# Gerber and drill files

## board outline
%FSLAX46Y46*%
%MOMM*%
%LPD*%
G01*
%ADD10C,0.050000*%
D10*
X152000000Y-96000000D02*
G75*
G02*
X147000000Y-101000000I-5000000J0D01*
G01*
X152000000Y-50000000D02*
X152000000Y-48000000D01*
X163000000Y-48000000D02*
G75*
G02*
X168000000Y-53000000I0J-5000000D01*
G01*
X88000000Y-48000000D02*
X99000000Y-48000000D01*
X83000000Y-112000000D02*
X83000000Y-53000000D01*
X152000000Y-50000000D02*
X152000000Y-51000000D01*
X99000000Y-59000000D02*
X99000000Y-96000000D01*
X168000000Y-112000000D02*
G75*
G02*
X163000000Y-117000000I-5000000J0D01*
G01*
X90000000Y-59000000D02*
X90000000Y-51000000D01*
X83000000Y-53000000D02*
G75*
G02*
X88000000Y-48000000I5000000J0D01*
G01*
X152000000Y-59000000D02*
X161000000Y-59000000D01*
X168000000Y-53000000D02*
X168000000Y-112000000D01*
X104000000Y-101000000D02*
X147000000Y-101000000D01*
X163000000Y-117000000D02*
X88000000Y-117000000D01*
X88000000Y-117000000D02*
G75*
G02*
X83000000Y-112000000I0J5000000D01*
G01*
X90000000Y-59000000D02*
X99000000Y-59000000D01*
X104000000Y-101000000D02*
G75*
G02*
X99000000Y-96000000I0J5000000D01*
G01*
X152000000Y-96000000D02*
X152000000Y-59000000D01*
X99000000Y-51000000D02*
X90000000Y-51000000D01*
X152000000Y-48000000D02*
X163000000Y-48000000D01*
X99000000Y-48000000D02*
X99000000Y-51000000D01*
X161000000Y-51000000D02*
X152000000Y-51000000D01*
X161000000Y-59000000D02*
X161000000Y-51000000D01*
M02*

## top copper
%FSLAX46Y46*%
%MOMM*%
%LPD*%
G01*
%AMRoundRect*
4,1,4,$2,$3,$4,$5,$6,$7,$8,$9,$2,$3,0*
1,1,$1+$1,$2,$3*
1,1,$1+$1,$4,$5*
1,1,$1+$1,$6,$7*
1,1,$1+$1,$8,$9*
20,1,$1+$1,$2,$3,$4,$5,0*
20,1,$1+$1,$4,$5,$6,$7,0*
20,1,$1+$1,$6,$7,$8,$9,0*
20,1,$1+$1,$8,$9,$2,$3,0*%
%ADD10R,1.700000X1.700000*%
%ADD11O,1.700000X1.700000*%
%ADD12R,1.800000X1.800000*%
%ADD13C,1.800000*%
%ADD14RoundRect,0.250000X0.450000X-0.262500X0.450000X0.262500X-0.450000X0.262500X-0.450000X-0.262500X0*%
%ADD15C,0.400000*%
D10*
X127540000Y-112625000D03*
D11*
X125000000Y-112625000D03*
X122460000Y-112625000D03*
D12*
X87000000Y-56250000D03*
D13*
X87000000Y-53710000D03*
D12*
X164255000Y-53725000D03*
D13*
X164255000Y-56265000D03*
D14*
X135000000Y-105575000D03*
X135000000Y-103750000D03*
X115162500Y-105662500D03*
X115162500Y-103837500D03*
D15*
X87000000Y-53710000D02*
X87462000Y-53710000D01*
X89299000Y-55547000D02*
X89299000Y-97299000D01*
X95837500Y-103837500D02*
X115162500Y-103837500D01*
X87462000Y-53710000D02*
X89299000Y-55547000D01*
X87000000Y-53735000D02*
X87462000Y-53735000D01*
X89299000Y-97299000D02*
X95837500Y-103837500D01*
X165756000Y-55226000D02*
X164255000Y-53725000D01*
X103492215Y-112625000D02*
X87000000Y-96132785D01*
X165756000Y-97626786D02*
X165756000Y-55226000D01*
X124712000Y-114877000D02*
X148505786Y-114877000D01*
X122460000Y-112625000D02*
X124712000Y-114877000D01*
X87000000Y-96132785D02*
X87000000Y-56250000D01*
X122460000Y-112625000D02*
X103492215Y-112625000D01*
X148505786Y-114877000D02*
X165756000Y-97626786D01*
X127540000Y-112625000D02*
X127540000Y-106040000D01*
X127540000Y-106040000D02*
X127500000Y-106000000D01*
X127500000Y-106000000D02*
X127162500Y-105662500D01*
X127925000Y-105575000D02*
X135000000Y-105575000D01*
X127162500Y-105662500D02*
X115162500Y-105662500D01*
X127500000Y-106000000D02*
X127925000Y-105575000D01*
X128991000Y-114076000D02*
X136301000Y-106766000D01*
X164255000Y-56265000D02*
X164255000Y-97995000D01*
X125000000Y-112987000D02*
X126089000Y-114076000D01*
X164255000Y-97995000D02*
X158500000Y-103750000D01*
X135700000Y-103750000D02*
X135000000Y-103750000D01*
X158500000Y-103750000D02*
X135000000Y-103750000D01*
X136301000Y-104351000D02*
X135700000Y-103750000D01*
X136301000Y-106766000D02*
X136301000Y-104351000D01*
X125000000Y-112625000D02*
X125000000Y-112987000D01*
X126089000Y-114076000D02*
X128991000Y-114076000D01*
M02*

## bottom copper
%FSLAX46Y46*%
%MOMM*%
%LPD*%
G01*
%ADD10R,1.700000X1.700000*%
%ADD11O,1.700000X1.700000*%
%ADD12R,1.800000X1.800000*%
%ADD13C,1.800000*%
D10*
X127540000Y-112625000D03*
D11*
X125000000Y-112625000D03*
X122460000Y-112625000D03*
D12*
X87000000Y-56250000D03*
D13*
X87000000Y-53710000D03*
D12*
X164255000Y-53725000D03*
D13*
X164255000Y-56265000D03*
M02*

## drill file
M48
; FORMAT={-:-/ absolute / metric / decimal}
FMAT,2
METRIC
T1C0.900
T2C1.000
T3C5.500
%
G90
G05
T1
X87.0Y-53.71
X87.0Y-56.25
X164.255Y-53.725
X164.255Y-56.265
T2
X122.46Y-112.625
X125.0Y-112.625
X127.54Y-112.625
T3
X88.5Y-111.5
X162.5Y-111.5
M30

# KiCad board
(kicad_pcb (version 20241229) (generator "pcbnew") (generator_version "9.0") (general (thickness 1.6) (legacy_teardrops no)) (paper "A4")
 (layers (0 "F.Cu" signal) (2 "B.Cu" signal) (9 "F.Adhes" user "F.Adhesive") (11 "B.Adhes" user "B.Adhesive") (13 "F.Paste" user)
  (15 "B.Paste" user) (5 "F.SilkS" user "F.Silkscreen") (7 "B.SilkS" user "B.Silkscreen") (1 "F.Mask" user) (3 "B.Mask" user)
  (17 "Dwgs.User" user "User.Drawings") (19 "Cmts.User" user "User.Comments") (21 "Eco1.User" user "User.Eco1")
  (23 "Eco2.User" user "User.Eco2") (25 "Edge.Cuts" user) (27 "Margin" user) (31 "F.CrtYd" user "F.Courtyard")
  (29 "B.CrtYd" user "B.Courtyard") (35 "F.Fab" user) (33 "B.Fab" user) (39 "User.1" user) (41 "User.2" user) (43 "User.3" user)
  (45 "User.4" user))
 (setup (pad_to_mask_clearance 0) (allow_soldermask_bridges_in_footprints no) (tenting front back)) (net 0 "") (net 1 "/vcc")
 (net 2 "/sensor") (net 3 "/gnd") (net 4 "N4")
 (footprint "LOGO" (layer "F.Cu") (at 92.75 75.25 90)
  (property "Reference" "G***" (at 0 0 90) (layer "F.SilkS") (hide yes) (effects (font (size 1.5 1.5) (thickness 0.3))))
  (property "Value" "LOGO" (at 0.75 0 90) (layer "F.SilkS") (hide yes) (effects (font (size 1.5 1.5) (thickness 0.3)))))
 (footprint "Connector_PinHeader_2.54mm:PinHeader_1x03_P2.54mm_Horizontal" (layer "F.Cu") (at 127.54 112.625 -90)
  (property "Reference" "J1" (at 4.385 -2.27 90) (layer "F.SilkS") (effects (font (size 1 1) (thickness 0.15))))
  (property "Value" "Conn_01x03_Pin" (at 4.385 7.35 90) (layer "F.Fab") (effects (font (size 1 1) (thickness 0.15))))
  (pad "1" thru_hole rect (at 0 0 270) (size 1.7 1.7) (drill 1) (layers "*.Cu" "*.Mask") (remove_unused_layers no) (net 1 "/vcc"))
  (pad "2" thru_hole oval (at 0 2.54 270) (size 1.7 1.7) (drill 1) (layers "*.Cu" "*.Mask") (remove_unused_layers no) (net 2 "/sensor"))
  (pad "3" thru_hole oval (at 0 5.08 270) (size 1.7 1.7) (drill 1) (layers "*.Cu" "*.Mask") (remove_unused_layers no) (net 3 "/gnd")))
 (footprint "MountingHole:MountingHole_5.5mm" (layer "F.Cu") (at 88.5 111.5)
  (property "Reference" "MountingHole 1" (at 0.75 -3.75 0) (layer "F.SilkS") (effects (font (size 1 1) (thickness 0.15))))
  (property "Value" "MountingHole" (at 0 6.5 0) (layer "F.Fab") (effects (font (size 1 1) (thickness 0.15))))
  (pad "" np_thru_hole circle (at 0 0) (size 5.5 5.5) (drill 5.5) (layers "*.Cu" "*.Mask")))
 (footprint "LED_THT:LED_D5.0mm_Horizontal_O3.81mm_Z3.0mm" (layer "F.Cu") (at 87 56.25 90)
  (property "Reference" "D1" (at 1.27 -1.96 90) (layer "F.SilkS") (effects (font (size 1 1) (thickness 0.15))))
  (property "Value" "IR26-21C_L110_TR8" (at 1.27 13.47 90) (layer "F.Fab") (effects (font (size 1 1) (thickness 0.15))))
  (pad "1" thru_hole rect (at 0 0 90) (size 1.8 1.8) (drill 0.9) (layers "*.Cu" "*.Mask") (remove_unused_layers no) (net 3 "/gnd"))
  (pad "2" thru_hole circle (at 2.54 0 90) (size 1.8 1.8) (drill 0.9) (layers "*.Cu" "*.Mask") (remove_unused_layers no) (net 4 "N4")))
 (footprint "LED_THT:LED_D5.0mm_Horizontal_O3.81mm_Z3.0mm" (layer "F.Cu") (at 164.255 53.725 -90)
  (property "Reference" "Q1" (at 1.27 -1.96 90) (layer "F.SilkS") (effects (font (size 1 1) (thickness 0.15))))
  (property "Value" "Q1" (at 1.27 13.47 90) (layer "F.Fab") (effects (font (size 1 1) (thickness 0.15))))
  (pad "1" thru_hole rect (at 0 0 270) (size 1.8 1.8) (drill 0.9) (layers "*.Cu" "*.Mask") (remove_unused_layers no) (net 3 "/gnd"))
  (pad "2" thru_hole circle (at 2.54 0 270) (size 1.8 1.8) (drill 0.9) (layers "*.Cu" "*.Mask") (remove_unused_layers no) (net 2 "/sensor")))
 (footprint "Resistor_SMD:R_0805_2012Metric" (layer "F.Cu") (at 135 104.6625 90)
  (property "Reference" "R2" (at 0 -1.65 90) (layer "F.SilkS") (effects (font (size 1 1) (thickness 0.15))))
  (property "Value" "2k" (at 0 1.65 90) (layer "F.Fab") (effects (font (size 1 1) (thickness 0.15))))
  (pad "1" smd roundrect (at -0.9125 0 90) (size 1.025 1.4) (layers "F.Cu" "F.Mask" "F.Paste") (roundrect_rratio 0.243902) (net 1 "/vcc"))
  (pad "2" smd roundrect (at 0.9125 0 90) (size 1.025 1.4) (layers "F.Cu" "F.Mask" "F.Paste") (roundrect_rratio 0.243902) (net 2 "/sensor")))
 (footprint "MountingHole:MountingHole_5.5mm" (layer "F.Cu") (at 162.5 111.5)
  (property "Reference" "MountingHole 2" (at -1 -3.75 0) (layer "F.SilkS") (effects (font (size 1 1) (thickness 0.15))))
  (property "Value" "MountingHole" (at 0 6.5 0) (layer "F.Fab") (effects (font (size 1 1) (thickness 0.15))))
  (pad "" np_thru_hole circle (at 0 0) (size 5.5 5.5) (drill 5.5) (layers "*.Cu" "*.Mask")))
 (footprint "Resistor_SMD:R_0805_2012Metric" (layer "F.Cu") (at 115.1625 104.75 90)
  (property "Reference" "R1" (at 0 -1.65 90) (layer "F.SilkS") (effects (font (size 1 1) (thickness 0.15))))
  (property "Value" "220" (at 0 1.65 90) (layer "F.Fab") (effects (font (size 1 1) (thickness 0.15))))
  (pad "1" smd roundrect (at -0.9125 0 90) (size 1.025 1.4) (layers "F.Cu" "F.Mask" "F.Paste") (roundrect_rratio 0.243902) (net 1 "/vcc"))
  (pad "2" smd roundrect (at 0.9125 0 90) (size 1.025 1.4) (layers "F.Cu" "F.Mask" "F.Paste") (roundrect_rratio 0.243902) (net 4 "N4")))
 (gr_arc (start 152 96) (mid 150.535534 99.535534) (end 147 101) (stroke (width 0.05) (type default)) (layer "Edge.Cuts"))
 (gr_line (start 152 50) (end 152 48) (stroke (width 0.05) (type default)) (layer "Edge.Cuts"))
 (gr_arc (start 163 48) (mid 166.535534 49.464466) (end 168 53) (stroke (width 0.05) (type default)) (layer "Edge.Cuts"))
 (gr_line (start 88 48) (end 99 48) (stroke (width 0.05) (type default)) (layer "Edge.Cuts"))
 (gr_line (start 83 112) (end 83 53) (stroke (width 0.05) (type default)) (layer "Edge.Cuts"))
 (gr_line (start 152 50) (end 152 51) (stroke (width 0.05) (type default)) (layer "Edge.Cuts"))
 (gr_line (start 99 59) (end 99 96) (stroke (width 0.05) (type default)) (layer "Edge.Cuts"))
 (gr_arc (start 168 112) (mid 166.535534 115.535534) (end 163 117) (stroke (width 0.05) (type default)) (layer "Edge.Cuts"))
 (gr_line (start 90 59) (end 90 51) (stroke (width 0.05) (type default)) (layer "Edge.Cuts"))
 (gr_arc (start 83 53) (mid 84.464466 49.464466) (end 88 48) (stroke (width 0.05) (type default)) (layer "Edge.Cuts"))
 (gr_line (start 152 59) (end 161 59) (stroke (width 0.05) (type default)) (layer "Edge.Cuts"))
 (gr_line (start 168 53) (end 168 112) (stroke (width 0.05) (type default)) (layer "Edge.Cuts"))
 (gr_line (start 104 101) (end 147 101) (stroke (width 0.05) (type default)) (layer "Edge.Cuts"))
 (gr_line (start 163 117) (end 88 117) (stroke (width 0.05) (type default)) (layer "Edge.Cuts"))
 (gr_arc (start 88 117) (mid 84.464466 115.535534) (end 83 112) (stroke (width 0.05) (type default)) (layer "Edge.Cuts"))
 (gr_line (start 90 59) (end 99 59) (stroke (width 0.05) (type default)) (layer "Edge.Cuts"))
 (gr_arc (start 104 101) (mid 100.464466 99.535534) (end 99 96) (stroke (width 0.05) (type default)) (layer "Edge.Cuts"))
 (gr_line (start 152 96) (end 152 59) (stroke (width 0.05) (type default)) (layer "Edge.Cuts"))
 (gr_line (start 99 51) (end 90 51) (stroke (width 0.05) (type default)) (layer "Edge.Cuts"))
 (gr_line (start 152 48) (end 163 48) (stroke (width 0.05) (type default)) (layer "Edge.Cuts"))
 (gr_line (start 99 48) (end 99 51) (stroke (width 0.05) (type default)) (layer "Edge.Cuts"))
 (gr_line (start 161 51) (end 152 51) (stroke (width 0.05) (type default)) (layer "Edge.Cuts"))
 (gr_line (start 161 59) (end 161 51) (stroke (width 0.05) (type default)) (layer "Edge.Cuts"))
 (segment (start 87 53.71) (end 87.462 53.71) (width 0.4) (layer "F.Cu") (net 4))
 (segment (start 89.299 55.547) (end 89.299 97.299) (width 0.4) (layer "F.Cu") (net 4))
 (segment (start 95.8375 103.8375) (end 115.1625 103.8375) (width 0.4) (layer "F.Cu") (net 4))
 (segment (start 87.462 53.71) (end 89.299 55.547) (width 0.4) (layer "F.Cu") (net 4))
 (segment (start 87 53.735) (end 87.462 53.735) (width 0.4) (layer "F.Cu") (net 4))
 (segment (start 89.299 97.299) (end 95.8375 103.8375) (width 0.4) (layer "F.Cu") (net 4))
 (segment (start 165.756 55.226) (end 164.255 53.725) (width 0.4) (layer "F.Cu") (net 3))
 (segment (start 103.492215 112.625) (end 87 96.132785) (width 0.4) (layer "F.Cu") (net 3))
 (segment (start 165.756 97.626786) (end 165.756 55.226) (width 0.4) (layer "F.Cu") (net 3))
 (segment (start 124.712 114.877) (end 148.505786 114.877) (width 0.4) (layer "F.Cu") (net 3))
 (segment (start 122.46 112.625) (end 124.712 114.877) (width 0.4) (layer "F.Cu") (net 3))
 (segment (start 87 96.132785) (end 87 56.25) (width 0.4) (layer "F.Cu") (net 3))
 (segment (start 122.46 112.625) (end 103.492215 112.625) (width 0.4) (layer "F.Cu") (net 3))
 (segment (start 148.505786 114.877) (end 165.756 97.626786) (width 0.4) (layer "F.Cu") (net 3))
 (segment (start 127.54 112.625) (end 127.54 106.04) (width 0.4) (layer "F.Cu") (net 1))
 (segment (start 127.54 106.04) (end 127.5 106) (width 0.4) (layer "F.Cu") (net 1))
 (segment (start 127.5 106) (end 127.1625 105.6625) (width 0.4) (layer "F.Cu") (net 1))
 (segment (start 127.925 105.575) (end 135 105.575) (width 0.4) (layer "F.Cu") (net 1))
 (segment (start 127.1625 105.6625) (end 115.1625 105.6625) (width 0.4) (layer "F.Cu") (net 1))
 (segment (start 127.5 106) (end 127.925 105.575) (width 0.4) (layer "F.Cu") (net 1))
 (segment (start 128.991 114.076) (end 136.301 106.766) (width 0.4) (layer "F.Cu") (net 2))
 (segment (start 164.255 56.265) (end 164.255 97.995) (width 0.4) (layer "F.Cu") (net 2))
 (segment (start 125 112.987) (end 126.089 114.076) (width 0.4) (layer "F.Cu") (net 2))
 (segment (start 164.255 97.995) (end 158.5 103.75) (width 0.4) (layer "F.Cu") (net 2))
 (segment (start 135.7 103.75) (end 135 103.75) (width 0.4) (layer "F.Cu") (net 2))
 (segment (start 158.5 103.75) (end 135 103.75) (width 0.4) (layer "F.Cu") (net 2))
 (segment (start 136.301 104.351) (end 135.7 103.75) (width 0.4) (layer "F.Cu") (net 2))
 (segment (start 136.301 106.766) (end 136.301 104.351) (width 0.4) (layer "F.Cu") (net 2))
 (segment (start 125 112.625) (end 125 112.987) (width 0.4) (layer "F.Cu") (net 2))
 (segment (start 126.089 114.076) (end 128.991 114.076) (width 0.4) (layer "F.Cu") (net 2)))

